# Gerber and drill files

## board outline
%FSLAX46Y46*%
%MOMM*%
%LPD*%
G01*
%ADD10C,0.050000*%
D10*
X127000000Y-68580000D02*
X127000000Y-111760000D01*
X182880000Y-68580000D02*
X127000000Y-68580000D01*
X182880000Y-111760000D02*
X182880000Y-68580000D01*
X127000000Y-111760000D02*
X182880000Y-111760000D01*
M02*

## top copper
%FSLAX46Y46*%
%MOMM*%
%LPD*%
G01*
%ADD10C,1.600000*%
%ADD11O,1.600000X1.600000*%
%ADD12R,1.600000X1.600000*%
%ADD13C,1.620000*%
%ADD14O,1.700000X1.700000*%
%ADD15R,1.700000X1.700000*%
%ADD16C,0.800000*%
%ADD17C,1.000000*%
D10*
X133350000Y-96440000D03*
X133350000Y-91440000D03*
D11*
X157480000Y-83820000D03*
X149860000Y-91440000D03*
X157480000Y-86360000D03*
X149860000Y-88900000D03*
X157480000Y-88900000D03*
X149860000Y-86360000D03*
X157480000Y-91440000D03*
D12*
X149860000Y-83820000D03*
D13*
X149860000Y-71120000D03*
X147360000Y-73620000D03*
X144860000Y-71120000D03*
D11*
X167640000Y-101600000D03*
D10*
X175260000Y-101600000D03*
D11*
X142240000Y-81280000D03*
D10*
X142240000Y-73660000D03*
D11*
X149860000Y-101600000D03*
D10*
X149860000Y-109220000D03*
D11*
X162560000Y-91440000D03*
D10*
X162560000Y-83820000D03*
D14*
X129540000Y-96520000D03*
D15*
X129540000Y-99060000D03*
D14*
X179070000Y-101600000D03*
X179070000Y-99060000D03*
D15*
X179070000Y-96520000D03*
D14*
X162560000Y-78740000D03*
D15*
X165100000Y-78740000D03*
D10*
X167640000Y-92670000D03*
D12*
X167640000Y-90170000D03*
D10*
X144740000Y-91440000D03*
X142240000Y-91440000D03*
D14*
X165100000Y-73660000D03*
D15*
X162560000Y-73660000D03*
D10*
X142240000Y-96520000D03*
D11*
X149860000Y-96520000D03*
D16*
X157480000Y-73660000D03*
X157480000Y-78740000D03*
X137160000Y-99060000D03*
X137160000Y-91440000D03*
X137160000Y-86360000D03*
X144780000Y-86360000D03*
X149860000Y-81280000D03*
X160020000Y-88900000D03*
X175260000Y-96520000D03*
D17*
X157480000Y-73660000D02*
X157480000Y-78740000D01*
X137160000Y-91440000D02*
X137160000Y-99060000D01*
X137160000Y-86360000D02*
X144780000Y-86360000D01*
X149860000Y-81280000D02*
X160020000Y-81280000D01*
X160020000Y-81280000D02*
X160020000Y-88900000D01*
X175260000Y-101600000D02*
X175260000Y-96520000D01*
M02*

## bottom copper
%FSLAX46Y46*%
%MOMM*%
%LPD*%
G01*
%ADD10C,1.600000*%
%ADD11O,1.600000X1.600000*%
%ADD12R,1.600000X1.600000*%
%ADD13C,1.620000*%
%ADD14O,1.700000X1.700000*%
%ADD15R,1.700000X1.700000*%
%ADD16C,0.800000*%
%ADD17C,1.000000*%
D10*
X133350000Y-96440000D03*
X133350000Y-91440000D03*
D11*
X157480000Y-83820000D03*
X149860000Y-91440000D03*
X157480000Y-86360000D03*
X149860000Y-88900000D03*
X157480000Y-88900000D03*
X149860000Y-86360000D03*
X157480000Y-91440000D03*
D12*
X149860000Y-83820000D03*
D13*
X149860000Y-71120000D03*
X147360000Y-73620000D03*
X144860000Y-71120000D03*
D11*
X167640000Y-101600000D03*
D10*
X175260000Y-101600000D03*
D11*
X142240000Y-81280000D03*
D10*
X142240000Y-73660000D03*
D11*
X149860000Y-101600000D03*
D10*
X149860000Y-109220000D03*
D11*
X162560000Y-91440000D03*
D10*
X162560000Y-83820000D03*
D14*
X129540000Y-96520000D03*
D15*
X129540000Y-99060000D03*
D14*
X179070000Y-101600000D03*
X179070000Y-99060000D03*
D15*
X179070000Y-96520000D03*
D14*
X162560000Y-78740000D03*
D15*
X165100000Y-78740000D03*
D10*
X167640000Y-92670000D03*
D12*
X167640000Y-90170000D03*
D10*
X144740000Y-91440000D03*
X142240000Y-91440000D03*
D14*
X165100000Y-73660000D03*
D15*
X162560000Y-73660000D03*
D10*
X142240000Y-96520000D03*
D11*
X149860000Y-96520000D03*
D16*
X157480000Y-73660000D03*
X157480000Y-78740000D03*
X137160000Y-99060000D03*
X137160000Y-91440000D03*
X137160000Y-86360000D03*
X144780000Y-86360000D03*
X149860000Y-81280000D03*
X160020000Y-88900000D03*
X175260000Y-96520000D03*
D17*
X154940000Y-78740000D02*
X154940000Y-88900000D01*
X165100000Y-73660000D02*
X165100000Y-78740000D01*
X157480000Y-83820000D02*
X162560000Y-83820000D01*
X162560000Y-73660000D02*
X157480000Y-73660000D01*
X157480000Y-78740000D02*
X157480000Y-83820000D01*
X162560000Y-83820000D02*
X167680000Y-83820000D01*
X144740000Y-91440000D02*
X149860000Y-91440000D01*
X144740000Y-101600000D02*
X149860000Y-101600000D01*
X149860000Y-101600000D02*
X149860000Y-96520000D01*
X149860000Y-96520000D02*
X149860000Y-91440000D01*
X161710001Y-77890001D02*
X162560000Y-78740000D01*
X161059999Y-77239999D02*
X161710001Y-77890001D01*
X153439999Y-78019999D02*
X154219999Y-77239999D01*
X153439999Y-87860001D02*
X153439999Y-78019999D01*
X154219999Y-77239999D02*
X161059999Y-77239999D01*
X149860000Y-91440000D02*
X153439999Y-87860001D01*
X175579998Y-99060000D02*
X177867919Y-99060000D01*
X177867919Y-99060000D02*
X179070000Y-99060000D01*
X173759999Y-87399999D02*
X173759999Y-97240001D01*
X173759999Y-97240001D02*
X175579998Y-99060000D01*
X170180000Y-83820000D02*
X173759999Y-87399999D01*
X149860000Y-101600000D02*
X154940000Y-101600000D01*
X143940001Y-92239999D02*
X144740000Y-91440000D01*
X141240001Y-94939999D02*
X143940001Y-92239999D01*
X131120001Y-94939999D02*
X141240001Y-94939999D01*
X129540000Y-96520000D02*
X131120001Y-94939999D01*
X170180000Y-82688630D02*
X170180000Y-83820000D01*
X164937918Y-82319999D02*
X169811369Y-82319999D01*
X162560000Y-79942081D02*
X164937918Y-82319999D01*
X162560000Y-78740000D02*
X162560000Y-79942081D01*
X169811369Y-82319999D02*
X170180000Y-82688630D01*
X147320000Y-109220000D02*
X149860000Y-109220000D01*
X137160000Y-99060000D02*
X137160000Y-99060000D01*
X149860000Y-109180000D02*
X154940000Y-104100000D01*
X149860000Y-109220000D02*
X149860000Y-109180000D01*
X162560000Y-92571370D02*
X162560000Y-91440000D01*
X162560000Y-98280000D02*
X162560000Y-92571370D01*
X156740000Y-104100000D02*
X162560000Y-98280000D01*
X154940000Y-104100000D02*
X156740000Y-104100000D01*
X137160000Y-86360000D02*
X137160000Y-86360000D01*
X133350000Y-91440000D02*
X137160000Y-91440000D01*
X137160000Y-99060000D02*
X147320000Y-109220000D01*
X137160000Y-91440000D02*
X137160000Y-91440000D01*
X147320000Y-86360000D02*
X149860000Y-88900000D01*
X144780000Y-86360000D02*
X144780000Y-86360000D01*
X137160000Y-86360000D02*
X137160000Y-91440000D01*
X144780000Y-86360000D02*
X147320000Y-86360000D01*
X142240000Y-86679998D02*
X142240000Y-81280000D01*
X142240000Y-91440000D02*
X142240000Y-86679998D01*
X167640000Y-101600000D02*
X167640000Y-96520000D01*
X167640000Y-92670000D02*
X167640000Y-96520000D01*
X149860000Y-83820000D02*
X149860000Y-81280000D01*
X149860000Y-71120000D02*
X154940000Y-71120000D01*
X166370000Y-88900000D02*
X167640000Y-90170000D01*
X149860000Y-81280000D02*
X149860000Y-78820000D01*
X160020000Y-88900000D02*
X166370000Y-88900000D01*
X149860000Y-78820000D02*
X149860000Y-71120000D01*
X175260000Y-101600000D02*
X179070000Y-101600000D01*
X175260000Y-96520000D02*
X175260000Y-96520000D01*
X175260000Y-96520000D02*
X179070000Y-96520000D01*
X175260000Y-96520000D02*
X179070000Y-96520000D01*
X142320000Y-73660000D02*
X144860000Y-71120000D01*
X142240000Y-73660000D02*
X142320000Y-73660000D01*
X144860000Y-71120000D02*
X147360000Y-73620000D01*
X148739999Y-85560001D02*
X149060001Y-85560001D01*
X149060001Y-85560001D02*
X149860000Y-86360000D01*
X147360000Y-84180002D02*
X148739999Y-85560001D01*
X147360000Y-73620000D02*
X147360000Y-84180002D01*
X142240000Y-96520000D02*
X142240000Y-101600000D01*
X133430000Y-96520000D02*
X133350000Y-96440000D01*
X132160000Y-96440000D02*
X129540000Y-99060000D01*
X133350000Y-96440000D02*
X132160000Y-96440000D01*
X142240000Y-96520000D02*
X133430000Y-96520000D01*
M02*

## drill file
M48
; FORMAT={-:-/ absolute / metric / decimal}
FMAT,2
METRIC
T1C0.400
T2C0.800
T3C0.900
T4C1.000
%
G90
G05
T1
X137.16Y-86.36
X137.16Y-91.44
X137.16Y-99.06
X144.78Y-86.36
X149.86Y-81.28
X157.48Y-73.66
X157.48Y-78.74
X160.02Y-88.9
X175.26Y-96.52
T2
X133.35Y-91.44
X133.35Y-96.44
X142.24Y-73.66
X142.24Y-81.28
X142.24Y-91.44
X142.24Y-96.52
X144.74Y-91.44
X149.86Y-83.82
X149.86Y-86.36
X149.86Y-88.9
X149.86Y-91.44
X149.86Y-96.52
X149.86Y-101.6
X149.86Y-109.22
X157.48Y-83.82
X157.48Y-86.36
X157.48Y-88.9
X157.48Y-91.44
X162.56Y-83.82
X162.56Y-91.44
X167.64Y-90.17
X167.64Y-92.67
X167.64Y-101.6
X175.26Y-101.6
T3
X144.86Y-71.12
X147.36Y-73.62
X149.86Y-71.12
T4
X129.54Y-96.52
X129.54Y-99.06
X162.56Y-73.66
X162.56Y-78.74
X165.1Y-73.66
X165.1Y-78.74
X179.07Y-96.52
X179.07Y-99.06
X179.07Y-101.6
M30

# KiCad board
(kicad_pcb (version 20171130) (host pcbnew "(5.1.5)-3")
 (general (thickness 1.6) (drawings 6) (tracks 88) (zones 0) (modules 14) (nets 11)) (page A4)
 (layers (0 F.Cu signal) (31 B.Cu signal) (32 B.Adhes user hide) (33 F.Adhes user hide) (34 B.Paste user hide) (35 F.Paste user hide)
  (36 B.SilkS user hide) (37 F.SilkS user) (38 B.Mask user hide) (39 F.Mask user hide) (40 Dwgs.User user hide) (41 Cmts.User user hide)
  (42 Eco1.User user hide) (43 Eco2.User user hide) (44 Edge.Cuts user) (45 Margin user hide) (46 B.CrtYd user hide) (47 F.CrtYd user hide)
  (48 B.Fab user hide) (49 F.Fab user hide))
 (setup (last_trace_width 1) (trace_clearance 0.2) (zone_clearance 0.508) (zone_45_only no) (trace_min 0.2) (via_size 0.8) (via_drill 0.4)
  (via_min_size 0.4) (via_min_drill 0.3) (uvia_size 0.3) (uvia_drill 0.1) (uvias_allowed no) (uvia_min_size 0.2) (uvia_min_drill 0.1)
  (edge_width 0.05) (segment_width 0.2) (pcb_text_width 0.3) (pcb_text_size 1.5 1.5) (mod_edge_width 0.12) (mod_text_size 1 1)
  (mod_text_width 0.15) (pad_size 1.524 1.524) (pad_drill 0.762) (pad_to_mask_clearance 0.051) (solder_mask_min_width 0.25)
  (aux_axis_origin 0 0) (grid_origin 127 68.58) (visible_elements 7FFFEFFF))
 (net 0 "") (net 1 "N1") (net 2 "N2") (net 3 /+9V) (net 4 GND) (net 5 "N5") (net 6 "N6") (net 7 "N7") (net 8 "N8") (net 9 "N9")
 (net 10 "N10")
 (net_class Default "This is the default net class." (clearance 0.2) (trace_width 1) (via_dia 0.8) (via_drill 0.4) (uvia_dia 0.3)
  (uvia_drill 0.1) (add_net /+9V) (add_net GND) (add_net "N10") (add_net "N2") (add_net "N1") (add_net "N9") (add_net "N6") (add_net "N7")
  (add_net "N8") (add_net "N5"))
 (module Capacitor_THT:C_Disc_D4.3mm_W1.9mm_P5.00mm (layer F.Cu) (at 133.35 91.44 270)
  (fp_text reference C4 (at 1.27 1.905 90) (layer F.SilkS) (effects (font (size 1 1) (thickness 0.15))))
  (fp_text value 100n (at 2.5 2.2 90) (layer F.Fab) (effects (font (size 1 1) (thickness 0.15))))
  (pad 2 thru_hole circle (at 5 0 270) (size 1.6 1.6) (drill 0.8) (layers *.Cu *.Mask) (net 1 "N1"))
  (pad 1 thru_hole circle (at 0 0 270) (size 1.6 1.6) (drill 0.8) (layers *.Cu *.Mask) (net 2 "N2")))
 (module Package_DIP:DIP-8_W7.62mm (layer F.Cu) (at 149.86 83.82)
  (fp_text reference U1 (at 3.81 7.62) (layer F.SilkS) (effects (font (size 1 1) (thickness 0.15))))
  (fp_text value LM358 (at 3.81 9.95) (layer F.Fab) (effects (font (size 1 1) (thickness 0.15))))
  (pad 8 thru_hole oval (at 7.62 0) (size 1.6 1.6) (drill 0.8) (layers *.Cu *.Mask) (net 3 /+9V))
  (pad 4 thru_hole oval (at 0 7.62) (size 1.6 1.6) (drill 0.8) (layers *.Cu *.Mask) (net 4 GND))
  (pad 7 thru_hole oval (at 7.62 2.54) (size 1.6 1.6) (drill 0.8) (layers *.Cu *.Mask))
  (pad 3 thru_hole oval (at 0 5.08) (size 1.6 1.6) (drill 0.8) (layers *.Cu *.Mask) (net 2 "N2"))
  (pad 6 thru_hole oval (at 7.62 5.08) (size 1.6 1.6) (drill 0.8) (layers *.Cu *.Mask))
  (pad 2 thru_hole oval (at 0 2.54) (size 1.6 1.6) (drill 0.8) (layers *.Cu *.Mask) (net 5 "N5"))
  (pad 5 thru_hole oval (at 7.62 7.62) (size 1.6 1.6) (drill 0.8) (layers *.Cu *.Mask))
  (pad 1 thru_hole rect (at 0 0) (size 1.6 1.6) (drill 0.8) (layers *.Cu *.Mask) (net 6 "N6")))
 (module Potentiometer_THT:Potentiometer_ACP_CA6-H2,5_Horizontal (layer F.Cu) (at 149.86 71.12 270)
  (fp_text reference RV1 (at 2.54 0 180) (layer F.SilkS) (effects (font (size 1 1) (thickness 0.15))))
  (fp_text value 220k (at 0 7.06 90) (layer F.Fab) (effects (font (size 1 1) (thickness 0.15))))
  (pad 1 thru_hole circle (at 0 0 270) (size 1.62 1.62) (drill 0.9) (layers *.Cu *.Mask) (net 6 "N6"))
  (pad 2 thru_hole circle (at 2.5 2.5 270) (size 1.62 1.62) (drill 0.9) (layers *.Cu *.Mask) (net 5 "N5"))
  (pad 3 thru_hole circle (at 0 5 270) (size 1.62 1.62) (drill 0.9) (layers *.Cu *.Mask) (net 5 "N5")))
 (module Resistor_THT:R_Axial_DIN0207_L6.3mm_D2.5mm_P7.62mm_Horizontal (layer F.Cu) (at 175.26 101.6 180)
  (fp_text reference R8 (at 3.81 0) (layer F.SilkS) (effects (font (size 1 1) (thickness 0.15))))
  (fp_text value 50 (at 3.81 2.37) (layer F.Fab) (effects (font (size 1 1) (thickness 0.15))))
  (pad 2 thru_hole oval (at 7.62 0 180) (size 1.6 1.6) (drill 0.8) (layers *.Cu *.Mask) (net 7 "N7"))
  (pad 1 thru_hole circle (at 0 0 180) (size 1.6 1.6) (drill 0.8) (layers *.Cu *.Mask) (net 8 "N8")))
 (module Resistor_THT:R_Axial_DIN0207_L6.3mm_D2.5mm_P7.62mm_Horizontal (layer F.Cu) (at 142.24 73.66 270)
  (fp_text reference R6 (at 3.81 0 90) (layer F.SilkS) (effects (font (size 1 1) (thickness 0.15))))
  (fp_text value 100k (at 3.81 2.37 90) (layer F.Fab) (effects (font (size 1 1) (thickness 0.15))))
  (pad 2 thru_hole oval (at 7.62 0 270) (size 1.6 1.6) (drill 0.8) (layers *.Cu *.Mask) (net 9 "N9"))
  (pad 1 thru_hole circle (at 0 0 270) (size 1.6 1.6) (drill 0.8) (layers *.Cu *.Mask) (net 5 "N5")))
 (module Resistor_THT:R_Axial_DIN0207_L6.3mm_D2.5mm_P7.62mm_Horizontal (layer F.Cu) (at 149.86 109.22 90)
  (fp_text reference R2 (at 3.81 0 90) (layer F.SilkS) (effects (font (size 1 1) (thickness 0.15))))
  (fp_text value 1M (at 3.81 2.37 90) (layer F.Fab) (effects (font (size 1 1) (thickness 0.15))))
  (pad 2 thru_hole oval (at 7.62 0 90) (size 1.6 1.6) (drill 0.8) (layers *.Cu *.Mask) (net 4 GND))
  (pad 1 thru_hole circle (at 0 0 90) (size 1.6 1.6) (drill 0.8) (layers *.Cu *.Mask) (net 2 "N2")))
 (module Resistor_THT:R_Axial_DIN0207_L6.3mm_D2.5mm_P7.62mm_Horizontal (layer F.Cu) (at 162.56 83.82 270)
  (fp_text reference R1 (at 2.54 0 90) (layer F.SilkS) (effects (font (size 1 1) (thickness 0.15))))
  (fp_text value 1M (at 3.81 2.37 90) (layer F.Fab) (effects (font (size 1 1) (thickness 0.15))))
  (pad 2 thru_hole oval (at 7.62 0 270) (size 1.6 1.6) (drill 0.8) (layers *.Cu *.Mask) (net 2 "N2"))
  (pad 1 thru_hole circle (at 0 0 270) (size 1.6 1.6) (drill 0.8) (layers *.Cu *.Mask) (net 3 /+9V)))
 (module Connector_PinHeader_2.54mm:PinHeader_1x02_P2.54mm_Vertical (layer F.Cu) (at 129.54 99.06 180)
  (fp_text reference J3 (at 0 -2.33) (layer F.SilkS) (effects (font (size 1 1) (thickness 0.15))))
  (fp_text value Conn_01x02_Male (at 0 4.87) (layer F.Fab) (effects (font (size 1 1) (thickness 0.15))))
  (pad 2 thru_hole oval (at 0 2.54 180) (size 1.7 1.7) (drill 1) (layers *.Cu *.Mask) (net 4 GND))
  (pad 1 thru_hole rect (at 0 0 180) (size 1.7 1.7) (drill 1) (layers *.Cu *.Mask) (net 1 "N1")))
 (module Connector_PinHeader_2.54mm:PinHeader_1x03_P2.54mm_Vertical (layer F.Cu) (at 179.07 96.52)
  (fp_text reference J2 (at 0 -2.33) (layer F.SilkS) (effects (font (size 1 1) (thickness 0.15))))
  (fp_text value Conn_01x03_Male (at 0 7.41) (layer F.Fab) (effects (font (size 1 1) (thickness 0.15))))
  (pad 3 thru_hole oval (at 0 5.08) (size 1.7 1.7) (drill 1) (layers *.Cu *.Mask) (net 8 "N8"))
  (pad 2 thru_hole oval (at 0 2.54) (size 1.7 1.7) (drill 1) (layers *.Cu *.Mask) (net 4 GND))
  (pad 1 thru_hole rect (at 0 0) (size 1.7 1.7) (drill 1) (layers *.Cu *.Mask) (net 8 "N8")))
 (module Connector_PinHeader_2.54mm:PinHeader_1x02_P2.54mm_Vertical (layer F.Cu) (at 165.1 78.74 270)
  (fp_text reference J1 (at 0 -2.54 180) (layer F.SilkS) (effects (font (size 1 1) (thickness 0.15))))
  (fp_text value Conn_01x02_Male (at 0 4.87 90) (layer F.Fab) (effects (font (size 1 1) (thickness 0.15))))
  (pad 2 thru_hole oval (at 0 2.54 270) (size 1.7 1.7) (drill 1) (layers *.Cu *.Mask) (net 4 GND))
  (pad 1 thru_hole rect (at 0 0 270) (size 1.7 1.7) (drill 1) (layers *.Cu *.Mask) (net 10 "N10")))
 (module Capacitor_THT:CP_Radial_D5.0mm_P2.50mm (layer F.Cu) (at 167.64 90.17 270)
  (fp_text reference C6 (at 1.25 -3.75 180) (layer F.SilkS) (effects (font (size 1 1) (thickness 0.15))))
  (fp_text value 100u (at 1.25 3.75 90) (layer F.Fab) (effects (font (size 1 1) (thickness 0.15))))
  (pad 2 thru_hole circle (at 2.5 0 270) (size 1.6 1.6) (drill 0.8) (layers *.Cu *.Mask) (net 7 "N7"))
  (pad 1 thru_hole rect (at 0 0 270) (size 1.6 1.6) (drill 0.8) (layers *.Cu *.Mask) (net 6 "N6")))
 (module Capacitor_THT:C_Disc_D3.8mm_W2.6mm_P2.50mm (layer F.Cu) (at 142.24 91.44)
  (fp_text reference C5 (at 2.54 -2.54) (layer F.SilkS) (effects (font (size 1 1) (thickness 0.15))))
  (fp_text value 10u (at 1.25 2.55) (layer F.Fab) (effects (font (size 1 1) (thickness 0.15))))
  (pad 2 thru_hole circle (at 2.5 0) (size 1.6 1.6) (drill 0.8) (layers *.Cu *.Mask) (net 4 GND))
  (pad 1 thru_hole circle (at 0 0) (size 1.6 1.6) (drill 0.8) (layers *.Cu *.Mask) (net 9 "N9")))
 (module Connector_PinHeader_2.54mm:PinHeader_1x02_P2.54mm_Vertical (layer F.Cu) (at 162.56 73.66 90)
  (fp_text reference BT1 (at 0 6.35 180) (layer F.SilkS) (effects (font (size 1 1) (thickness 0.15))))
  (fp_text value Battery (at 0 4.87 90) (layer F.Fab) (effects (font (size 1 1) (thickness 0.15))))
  (pad 2 thru_hole oval (at 0 2.54 90) (size 1.7 1.7) (drill 1) (layers *.Cu *.Mask) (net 10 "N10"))
  (pad 1 thru_hole rect (at 0 0 90) (size 1.7 1.7) (drill 1) (layers *.Cu *.Mask) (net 3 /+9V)))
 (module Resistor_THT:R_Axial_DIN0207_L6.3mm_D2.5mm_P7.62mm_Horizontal (layer F.Cu) (at 142.24 96.52)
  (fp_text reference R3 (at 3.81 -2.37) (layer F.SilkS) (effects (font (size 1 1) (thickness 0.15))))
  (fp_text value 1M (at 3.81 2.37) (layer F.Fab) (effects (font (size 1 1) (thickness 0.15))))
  (pad 1 thru_hole circle (at 0 0) (size 1.6 1.6) (drill 0.8) (layers *.Cu *.Mask) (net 1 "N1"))
  (pad 2 thru_hole oval (at 7.62 0) (size 1.6 1.6) (drill 0.8) (layers *.Cu *.Mask) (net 4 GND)))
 (gr_line (start 127 68.58) (end 127 111.76) (layer Edge.Cuts) (width 0.05))
 (gr_line (start 182.88 68.58) (end 127 68.58) (layer Edge.Cuts) (width 0.05))
 (gr_line (start 182.88 111.76) (end 182.88 68.58) (layer Edge.Cuts) (width 0.05))
 (gr_line (start 127 111.76) (end 182.88 111.76) (layer Edge.Cuts) (width 0.05))
 (segment (start 154.94 78.74) (end 154.94 88.9) (width 1) (layer B.Cu) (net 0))
 (segment (start 165.1 73.66) (end 165.1 78.74) (width 1) (layer B.Cu) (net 10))
 (segment (start 157.48 83.82) (end 162.56 83.82) (width 1) (layer B.Cu) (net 3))
 (via (at 157.48 73.66) (size 0.8) (drill 0.4) (layers F.Cu B.Cu) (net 3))
 (segment (start 162.56 73.66) (end 157.48 73.66) (width 1) (layer B.Cu) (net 3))
 (via (at 157.48 78.74) (size 0.8) (drill 0.4) (layers F.Cu B.Cu) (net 3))
 (segment (start 157.48 73.66) (end 157.48 78.74) (width 1) (layer F.Cu) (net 3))
 (segment (start 157.48 78.74) (end 157.48 83.82) (width 1) (layer B.Cu) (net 3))
 (segment (start 162.56 83.82) (end 167.68 83.82) (width 1) (layer B.Cu) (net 3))
 (segment (start 144.74 91.44) (end 149.86 91.44) (width 1) (layer B.Cu) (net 4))
 (segment (start 144.74 101.6) (end 149.86 101.6) (width 1) (layer B.Cu) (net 4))
 (segment (start 149.86 101.6) (end 149.86 96.52) (width 1) (layer B.Cu) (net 4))
 (segment (start 149.86 96.52) (end 149.86 91.44) (width 1) (layer B.Cu) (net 4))
 (segment (start 161.710001 77.890001) (end 162.56 78.74) (width 1) (layer B.Cu) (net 4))
 (segment (start 161.059999 77.239999) (end 161.710001 77.890001) (width 1) (layer B.Cu) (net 4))
 (segment (start 153.439999 78.019999) (end 154.219999 77.239999) (width 1) (layer B.Cu) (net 4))
 (segment (start 153.439999 87.860001) (end 153.439999 78.019999) (width 1) (layer B.Cu) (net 4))
 (segment (start 154.219999 77.239999) (end 161.059999 77.239999) (width 1) (layer B.Cu) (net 4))
 (segment (start 149.86 91.44) (end 153.439999 87.860001) (width 1) (layer B.Cu) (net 4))
 (segment (start 175.579998 99.06) (end 177.867919 99.06) (width 1) (layer B.Cu) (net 4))
 (segment (start 177.867919 99.06) (end 179.07 99.06) (width 1) (layer B.Cu) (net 4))
 (segment (start 173.759999 87.399999) (end 173.759999 97.240001) (width 1) (layer B.Cu) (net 4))
 (segment (start 173.759999 97.240001) (end 175.579998 99.06) (width 1) (layer B.Cu) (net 4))
 (segment (start 170.18 83.82) (end 173.759999 87.399999) (width 1) (layer B.Cu) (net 4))
 (segment (start 149.86 101.6) (end 154.94 101.6) (width 1) (layer B.Cu) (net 4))
 (segment (start 143.940001 92.239999) (end 144.74 91.44) (width 1) (layer B.Cu) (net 4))
 (segment (start 141.240001 94.939999) (end 143.940001 92.239999) (width 1) (layer B.Cu) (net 4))
 (segment (start 131.120001 94.939999) (end 141.240001 94.939999) (width 1) (layer B.Cu) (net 4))
 (segment (start 129.54 96.52) (end 131.120001 94.939999) (width 1) (layer B.Cu) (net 4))
 (segment (start 170.18 82.68863) (end 170.18 83.82) (width 1) (layer B.Cu) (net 4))
 (segment (start 164.937918 82.319999) (end 169.811369 82.319999) (width 1) (layer B.Cu) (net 4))
 (segment (start 162.56 79.942081) (end 164.937918 82.319999) (width 1) (layer B.Cu) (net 4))
 (segment (start 162.56 78.74) (end 162.56 79.942081) (width 1) (layer B.Cu) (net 4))
 (segment (start 169.811369 82.319999) (end 170.18 82.68863) (width 1) (layer B.Cu) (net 4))
 (segment (start 147.32 109.22) (end 149.86 109.22) (width 1) (layer B.Cu) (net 2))
 (segment (start 137.16 99.06) (end 137.16 99.06) (width 1) (layer B.Cu) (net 2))
 (segment (start 149.86 109.18) (end 154.94 104.1) (width 1) (layer B.Cu) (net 2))
 (segment (start 149.86 109.22) (end 149.86 109.18) (width 1) (layer B.Cu) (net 2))
 (segment (start 162.56 92.57137) (end 162.56 91.44) (width 1) (layer B.Cu) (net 2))
 (segment (start 162.56 98.28) (end 162.56 92.57137) (width 1) (layer B.Cu) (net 2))
 (segment (start 156.74 104.1) (end 162.56 98.28) (width 1) (layer B.Cu) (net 2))
 (segment (start 154.94 104.1) (end 156.74 104.1) (width 1) (layer B.Cu) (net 2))
 (segment (start 137.16 86.36) (end 137.16 86.36) (width 1) (layer B.Cu) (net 2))
 (segment (start 133.35 91.44) (end 137.16 91.44) (width 1) (layer B.Cu) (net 2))
 (segment (start 137.16 99.06) (end 147.32 109.22) (width 1) (layer B.Cu) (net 2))
 (via (at 137.16 99.06) (size 0.8) (drill 0.4) (layers F.Cu B.Cu) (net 2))
 (segment (start 137.16 91.44) (end 137.16 91.44) (width 1) (layer B.Cu) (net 2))
 (via (at 137.16 91.44) (size 0.8) (drill 0.4) (layers F.Cu B.Cu) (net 2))
 (segment (start 137.16 91.44) (end 137.16 99.06) (width 1) (layer F.Cu) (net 2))
 (segment (start 147.32 86.36) (end 149.86 88.9) (width 1) (layer B.Cu) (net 2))
 (segment (start 144.78 86.36) (end 144.78 86.36) (width 1) (layer B.Cu) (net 2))
 (segment (start 137.16 86.36) (end 137.16 91.44) (width 1) (layer B.Cu) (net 2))
 (via (at 137.16 86.36) (size 0.8) (drill 0.4) (layers F.Cu B.Cu) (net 2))
 (segment (start 144.78 86.36) (end 147.32 86.36) (width 1) (layer B.Cu) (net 2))
 (via (at 144.78 86.36) (size 0.8) (drill 0.4) (layers F.Cu B.Cu) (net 2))
 (segment (start 137.16 86.36) (end 144.78 86.36) (width 1) (layer F.Cu) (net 2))
 (segment (start 142.24 86.679998) (end 142.24 81.28) (width 1) (layer B.Cu) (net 9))
 (segment (start 142.24 91.44) (end 142.24 86.679998) (width 1) (layer B.Cu) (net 9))
 (segment (start 167.64 101.6) (end 167.64 96.52) (width 1) (layer B.Cu) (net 7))
 (segment (start 167.64 92.67) (end 167.64 96.52) (width 1) (layer B.Cu) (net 7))
 (segment (start 149.86 83.82) (end 149.86 81.28) (width 1) (layer B.Cu) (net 6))
 (segment (start 149.86 71.12) (end 154.94 71.12) (width 1) (layer B.Cu) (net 6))
 (segment (start 166.37 88.9) (end 167.64 90.17) (width 1) (layer B.Cu) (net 6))
 (segment (start 149.86 81.28) (end 149.86 78.82) (width 1) (layer B.Cu) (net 6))
 (via (at 149.86 81.28) (size 0.8) (drill 0.4) (layers F.Cu B.Cu) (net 6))
 (segment (start 160.02 88.9) (end 166.37 88.9) (width 1) (layer B.Cu) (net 6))
 (via (at 160.02 88.9) (size 0.8) (drill 0.4) (layers F.Cu B.Cu) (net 6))
 (segment (start 149.86 81.28) (end 160.02 81.28) (width 1) (layer F.Cu) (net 6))
 (segment (start 160.02 81.28) (end 160.02 88.9) (width 1) (layer F.Cu) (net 6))
 (segment (start 149.86 78.82) (end 149.86 71.12) (width 1) (layer B.Cu) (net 6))
 (segment (start 175.26 101.6) (end 179.07 101.6) (width 1) (layer B.Cu) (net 8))
 (segment (start 175.26 96.52) (end 175.26 96.52) (width 1) (layer B.Cu) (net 8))
 (segment (start 175.26 96.52) (end 179.07 96.52) (width 1) (layer B.Cu) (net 8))
 (segment (start 175.26 101.6) (end 175.26 96.52) (width 1) (layer F.Cu) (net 8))
 (segment (start 175.26 96.52) (end 179.07 96.52) (width 1) (layer B.Cu) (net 8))
 (via (at 175.26 96.52) (size 0.8) (drill 0.4) (layers F.Cu B.Cu) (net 8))
 (segment (start 142.32 73.66) (end 144.86 71.12) (width 1) (layer B.Cu) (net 5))
 (segment (start 142.24 73.66) (end 142.32 73.66) (width 1) (layer B.Cu) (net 5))
 (segment (start 144.86 71.12) (end 147.36 73.62) (width 1) (layer B.Cu) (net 5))
 (segment (start 148.739999 85.560001) (end 149.060001 85.560001) (width 1) (layer B.Cu) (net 5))
 (segment (start 149.060001 85.560001) (end 149.86 86.36) (width 1) (layer B.Cu) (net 5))
 (segment (start 147.36 84.180002) (end 148.739999 85.560001) (width 1) (layer B.Cu) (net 5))
 (segment (start 147.36 73.62) (end 147.36 84.180002) (width 1) (layer B.Cu) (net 5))
 (segment (start 142.24 96.52) (end 142.24 101.6) (width 1) (layer B.Cu) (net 1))
 (segment (start 133.43 96.52) (end 133.35 96.44) (width 1) (layer B.Cu) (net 1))
 (segment (start 132.16 96.44) (end 129.54 99.06) (width 1) (layer B.Cu) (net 1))
 (segment (start 133.35 96.44) (end 132.16 96.44) (width 1) (layer B.Cu) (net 1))
 (segment (start 142.24 96.52) (end 133.43 96.52) (width 1) (layer B.Cu) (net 1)))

